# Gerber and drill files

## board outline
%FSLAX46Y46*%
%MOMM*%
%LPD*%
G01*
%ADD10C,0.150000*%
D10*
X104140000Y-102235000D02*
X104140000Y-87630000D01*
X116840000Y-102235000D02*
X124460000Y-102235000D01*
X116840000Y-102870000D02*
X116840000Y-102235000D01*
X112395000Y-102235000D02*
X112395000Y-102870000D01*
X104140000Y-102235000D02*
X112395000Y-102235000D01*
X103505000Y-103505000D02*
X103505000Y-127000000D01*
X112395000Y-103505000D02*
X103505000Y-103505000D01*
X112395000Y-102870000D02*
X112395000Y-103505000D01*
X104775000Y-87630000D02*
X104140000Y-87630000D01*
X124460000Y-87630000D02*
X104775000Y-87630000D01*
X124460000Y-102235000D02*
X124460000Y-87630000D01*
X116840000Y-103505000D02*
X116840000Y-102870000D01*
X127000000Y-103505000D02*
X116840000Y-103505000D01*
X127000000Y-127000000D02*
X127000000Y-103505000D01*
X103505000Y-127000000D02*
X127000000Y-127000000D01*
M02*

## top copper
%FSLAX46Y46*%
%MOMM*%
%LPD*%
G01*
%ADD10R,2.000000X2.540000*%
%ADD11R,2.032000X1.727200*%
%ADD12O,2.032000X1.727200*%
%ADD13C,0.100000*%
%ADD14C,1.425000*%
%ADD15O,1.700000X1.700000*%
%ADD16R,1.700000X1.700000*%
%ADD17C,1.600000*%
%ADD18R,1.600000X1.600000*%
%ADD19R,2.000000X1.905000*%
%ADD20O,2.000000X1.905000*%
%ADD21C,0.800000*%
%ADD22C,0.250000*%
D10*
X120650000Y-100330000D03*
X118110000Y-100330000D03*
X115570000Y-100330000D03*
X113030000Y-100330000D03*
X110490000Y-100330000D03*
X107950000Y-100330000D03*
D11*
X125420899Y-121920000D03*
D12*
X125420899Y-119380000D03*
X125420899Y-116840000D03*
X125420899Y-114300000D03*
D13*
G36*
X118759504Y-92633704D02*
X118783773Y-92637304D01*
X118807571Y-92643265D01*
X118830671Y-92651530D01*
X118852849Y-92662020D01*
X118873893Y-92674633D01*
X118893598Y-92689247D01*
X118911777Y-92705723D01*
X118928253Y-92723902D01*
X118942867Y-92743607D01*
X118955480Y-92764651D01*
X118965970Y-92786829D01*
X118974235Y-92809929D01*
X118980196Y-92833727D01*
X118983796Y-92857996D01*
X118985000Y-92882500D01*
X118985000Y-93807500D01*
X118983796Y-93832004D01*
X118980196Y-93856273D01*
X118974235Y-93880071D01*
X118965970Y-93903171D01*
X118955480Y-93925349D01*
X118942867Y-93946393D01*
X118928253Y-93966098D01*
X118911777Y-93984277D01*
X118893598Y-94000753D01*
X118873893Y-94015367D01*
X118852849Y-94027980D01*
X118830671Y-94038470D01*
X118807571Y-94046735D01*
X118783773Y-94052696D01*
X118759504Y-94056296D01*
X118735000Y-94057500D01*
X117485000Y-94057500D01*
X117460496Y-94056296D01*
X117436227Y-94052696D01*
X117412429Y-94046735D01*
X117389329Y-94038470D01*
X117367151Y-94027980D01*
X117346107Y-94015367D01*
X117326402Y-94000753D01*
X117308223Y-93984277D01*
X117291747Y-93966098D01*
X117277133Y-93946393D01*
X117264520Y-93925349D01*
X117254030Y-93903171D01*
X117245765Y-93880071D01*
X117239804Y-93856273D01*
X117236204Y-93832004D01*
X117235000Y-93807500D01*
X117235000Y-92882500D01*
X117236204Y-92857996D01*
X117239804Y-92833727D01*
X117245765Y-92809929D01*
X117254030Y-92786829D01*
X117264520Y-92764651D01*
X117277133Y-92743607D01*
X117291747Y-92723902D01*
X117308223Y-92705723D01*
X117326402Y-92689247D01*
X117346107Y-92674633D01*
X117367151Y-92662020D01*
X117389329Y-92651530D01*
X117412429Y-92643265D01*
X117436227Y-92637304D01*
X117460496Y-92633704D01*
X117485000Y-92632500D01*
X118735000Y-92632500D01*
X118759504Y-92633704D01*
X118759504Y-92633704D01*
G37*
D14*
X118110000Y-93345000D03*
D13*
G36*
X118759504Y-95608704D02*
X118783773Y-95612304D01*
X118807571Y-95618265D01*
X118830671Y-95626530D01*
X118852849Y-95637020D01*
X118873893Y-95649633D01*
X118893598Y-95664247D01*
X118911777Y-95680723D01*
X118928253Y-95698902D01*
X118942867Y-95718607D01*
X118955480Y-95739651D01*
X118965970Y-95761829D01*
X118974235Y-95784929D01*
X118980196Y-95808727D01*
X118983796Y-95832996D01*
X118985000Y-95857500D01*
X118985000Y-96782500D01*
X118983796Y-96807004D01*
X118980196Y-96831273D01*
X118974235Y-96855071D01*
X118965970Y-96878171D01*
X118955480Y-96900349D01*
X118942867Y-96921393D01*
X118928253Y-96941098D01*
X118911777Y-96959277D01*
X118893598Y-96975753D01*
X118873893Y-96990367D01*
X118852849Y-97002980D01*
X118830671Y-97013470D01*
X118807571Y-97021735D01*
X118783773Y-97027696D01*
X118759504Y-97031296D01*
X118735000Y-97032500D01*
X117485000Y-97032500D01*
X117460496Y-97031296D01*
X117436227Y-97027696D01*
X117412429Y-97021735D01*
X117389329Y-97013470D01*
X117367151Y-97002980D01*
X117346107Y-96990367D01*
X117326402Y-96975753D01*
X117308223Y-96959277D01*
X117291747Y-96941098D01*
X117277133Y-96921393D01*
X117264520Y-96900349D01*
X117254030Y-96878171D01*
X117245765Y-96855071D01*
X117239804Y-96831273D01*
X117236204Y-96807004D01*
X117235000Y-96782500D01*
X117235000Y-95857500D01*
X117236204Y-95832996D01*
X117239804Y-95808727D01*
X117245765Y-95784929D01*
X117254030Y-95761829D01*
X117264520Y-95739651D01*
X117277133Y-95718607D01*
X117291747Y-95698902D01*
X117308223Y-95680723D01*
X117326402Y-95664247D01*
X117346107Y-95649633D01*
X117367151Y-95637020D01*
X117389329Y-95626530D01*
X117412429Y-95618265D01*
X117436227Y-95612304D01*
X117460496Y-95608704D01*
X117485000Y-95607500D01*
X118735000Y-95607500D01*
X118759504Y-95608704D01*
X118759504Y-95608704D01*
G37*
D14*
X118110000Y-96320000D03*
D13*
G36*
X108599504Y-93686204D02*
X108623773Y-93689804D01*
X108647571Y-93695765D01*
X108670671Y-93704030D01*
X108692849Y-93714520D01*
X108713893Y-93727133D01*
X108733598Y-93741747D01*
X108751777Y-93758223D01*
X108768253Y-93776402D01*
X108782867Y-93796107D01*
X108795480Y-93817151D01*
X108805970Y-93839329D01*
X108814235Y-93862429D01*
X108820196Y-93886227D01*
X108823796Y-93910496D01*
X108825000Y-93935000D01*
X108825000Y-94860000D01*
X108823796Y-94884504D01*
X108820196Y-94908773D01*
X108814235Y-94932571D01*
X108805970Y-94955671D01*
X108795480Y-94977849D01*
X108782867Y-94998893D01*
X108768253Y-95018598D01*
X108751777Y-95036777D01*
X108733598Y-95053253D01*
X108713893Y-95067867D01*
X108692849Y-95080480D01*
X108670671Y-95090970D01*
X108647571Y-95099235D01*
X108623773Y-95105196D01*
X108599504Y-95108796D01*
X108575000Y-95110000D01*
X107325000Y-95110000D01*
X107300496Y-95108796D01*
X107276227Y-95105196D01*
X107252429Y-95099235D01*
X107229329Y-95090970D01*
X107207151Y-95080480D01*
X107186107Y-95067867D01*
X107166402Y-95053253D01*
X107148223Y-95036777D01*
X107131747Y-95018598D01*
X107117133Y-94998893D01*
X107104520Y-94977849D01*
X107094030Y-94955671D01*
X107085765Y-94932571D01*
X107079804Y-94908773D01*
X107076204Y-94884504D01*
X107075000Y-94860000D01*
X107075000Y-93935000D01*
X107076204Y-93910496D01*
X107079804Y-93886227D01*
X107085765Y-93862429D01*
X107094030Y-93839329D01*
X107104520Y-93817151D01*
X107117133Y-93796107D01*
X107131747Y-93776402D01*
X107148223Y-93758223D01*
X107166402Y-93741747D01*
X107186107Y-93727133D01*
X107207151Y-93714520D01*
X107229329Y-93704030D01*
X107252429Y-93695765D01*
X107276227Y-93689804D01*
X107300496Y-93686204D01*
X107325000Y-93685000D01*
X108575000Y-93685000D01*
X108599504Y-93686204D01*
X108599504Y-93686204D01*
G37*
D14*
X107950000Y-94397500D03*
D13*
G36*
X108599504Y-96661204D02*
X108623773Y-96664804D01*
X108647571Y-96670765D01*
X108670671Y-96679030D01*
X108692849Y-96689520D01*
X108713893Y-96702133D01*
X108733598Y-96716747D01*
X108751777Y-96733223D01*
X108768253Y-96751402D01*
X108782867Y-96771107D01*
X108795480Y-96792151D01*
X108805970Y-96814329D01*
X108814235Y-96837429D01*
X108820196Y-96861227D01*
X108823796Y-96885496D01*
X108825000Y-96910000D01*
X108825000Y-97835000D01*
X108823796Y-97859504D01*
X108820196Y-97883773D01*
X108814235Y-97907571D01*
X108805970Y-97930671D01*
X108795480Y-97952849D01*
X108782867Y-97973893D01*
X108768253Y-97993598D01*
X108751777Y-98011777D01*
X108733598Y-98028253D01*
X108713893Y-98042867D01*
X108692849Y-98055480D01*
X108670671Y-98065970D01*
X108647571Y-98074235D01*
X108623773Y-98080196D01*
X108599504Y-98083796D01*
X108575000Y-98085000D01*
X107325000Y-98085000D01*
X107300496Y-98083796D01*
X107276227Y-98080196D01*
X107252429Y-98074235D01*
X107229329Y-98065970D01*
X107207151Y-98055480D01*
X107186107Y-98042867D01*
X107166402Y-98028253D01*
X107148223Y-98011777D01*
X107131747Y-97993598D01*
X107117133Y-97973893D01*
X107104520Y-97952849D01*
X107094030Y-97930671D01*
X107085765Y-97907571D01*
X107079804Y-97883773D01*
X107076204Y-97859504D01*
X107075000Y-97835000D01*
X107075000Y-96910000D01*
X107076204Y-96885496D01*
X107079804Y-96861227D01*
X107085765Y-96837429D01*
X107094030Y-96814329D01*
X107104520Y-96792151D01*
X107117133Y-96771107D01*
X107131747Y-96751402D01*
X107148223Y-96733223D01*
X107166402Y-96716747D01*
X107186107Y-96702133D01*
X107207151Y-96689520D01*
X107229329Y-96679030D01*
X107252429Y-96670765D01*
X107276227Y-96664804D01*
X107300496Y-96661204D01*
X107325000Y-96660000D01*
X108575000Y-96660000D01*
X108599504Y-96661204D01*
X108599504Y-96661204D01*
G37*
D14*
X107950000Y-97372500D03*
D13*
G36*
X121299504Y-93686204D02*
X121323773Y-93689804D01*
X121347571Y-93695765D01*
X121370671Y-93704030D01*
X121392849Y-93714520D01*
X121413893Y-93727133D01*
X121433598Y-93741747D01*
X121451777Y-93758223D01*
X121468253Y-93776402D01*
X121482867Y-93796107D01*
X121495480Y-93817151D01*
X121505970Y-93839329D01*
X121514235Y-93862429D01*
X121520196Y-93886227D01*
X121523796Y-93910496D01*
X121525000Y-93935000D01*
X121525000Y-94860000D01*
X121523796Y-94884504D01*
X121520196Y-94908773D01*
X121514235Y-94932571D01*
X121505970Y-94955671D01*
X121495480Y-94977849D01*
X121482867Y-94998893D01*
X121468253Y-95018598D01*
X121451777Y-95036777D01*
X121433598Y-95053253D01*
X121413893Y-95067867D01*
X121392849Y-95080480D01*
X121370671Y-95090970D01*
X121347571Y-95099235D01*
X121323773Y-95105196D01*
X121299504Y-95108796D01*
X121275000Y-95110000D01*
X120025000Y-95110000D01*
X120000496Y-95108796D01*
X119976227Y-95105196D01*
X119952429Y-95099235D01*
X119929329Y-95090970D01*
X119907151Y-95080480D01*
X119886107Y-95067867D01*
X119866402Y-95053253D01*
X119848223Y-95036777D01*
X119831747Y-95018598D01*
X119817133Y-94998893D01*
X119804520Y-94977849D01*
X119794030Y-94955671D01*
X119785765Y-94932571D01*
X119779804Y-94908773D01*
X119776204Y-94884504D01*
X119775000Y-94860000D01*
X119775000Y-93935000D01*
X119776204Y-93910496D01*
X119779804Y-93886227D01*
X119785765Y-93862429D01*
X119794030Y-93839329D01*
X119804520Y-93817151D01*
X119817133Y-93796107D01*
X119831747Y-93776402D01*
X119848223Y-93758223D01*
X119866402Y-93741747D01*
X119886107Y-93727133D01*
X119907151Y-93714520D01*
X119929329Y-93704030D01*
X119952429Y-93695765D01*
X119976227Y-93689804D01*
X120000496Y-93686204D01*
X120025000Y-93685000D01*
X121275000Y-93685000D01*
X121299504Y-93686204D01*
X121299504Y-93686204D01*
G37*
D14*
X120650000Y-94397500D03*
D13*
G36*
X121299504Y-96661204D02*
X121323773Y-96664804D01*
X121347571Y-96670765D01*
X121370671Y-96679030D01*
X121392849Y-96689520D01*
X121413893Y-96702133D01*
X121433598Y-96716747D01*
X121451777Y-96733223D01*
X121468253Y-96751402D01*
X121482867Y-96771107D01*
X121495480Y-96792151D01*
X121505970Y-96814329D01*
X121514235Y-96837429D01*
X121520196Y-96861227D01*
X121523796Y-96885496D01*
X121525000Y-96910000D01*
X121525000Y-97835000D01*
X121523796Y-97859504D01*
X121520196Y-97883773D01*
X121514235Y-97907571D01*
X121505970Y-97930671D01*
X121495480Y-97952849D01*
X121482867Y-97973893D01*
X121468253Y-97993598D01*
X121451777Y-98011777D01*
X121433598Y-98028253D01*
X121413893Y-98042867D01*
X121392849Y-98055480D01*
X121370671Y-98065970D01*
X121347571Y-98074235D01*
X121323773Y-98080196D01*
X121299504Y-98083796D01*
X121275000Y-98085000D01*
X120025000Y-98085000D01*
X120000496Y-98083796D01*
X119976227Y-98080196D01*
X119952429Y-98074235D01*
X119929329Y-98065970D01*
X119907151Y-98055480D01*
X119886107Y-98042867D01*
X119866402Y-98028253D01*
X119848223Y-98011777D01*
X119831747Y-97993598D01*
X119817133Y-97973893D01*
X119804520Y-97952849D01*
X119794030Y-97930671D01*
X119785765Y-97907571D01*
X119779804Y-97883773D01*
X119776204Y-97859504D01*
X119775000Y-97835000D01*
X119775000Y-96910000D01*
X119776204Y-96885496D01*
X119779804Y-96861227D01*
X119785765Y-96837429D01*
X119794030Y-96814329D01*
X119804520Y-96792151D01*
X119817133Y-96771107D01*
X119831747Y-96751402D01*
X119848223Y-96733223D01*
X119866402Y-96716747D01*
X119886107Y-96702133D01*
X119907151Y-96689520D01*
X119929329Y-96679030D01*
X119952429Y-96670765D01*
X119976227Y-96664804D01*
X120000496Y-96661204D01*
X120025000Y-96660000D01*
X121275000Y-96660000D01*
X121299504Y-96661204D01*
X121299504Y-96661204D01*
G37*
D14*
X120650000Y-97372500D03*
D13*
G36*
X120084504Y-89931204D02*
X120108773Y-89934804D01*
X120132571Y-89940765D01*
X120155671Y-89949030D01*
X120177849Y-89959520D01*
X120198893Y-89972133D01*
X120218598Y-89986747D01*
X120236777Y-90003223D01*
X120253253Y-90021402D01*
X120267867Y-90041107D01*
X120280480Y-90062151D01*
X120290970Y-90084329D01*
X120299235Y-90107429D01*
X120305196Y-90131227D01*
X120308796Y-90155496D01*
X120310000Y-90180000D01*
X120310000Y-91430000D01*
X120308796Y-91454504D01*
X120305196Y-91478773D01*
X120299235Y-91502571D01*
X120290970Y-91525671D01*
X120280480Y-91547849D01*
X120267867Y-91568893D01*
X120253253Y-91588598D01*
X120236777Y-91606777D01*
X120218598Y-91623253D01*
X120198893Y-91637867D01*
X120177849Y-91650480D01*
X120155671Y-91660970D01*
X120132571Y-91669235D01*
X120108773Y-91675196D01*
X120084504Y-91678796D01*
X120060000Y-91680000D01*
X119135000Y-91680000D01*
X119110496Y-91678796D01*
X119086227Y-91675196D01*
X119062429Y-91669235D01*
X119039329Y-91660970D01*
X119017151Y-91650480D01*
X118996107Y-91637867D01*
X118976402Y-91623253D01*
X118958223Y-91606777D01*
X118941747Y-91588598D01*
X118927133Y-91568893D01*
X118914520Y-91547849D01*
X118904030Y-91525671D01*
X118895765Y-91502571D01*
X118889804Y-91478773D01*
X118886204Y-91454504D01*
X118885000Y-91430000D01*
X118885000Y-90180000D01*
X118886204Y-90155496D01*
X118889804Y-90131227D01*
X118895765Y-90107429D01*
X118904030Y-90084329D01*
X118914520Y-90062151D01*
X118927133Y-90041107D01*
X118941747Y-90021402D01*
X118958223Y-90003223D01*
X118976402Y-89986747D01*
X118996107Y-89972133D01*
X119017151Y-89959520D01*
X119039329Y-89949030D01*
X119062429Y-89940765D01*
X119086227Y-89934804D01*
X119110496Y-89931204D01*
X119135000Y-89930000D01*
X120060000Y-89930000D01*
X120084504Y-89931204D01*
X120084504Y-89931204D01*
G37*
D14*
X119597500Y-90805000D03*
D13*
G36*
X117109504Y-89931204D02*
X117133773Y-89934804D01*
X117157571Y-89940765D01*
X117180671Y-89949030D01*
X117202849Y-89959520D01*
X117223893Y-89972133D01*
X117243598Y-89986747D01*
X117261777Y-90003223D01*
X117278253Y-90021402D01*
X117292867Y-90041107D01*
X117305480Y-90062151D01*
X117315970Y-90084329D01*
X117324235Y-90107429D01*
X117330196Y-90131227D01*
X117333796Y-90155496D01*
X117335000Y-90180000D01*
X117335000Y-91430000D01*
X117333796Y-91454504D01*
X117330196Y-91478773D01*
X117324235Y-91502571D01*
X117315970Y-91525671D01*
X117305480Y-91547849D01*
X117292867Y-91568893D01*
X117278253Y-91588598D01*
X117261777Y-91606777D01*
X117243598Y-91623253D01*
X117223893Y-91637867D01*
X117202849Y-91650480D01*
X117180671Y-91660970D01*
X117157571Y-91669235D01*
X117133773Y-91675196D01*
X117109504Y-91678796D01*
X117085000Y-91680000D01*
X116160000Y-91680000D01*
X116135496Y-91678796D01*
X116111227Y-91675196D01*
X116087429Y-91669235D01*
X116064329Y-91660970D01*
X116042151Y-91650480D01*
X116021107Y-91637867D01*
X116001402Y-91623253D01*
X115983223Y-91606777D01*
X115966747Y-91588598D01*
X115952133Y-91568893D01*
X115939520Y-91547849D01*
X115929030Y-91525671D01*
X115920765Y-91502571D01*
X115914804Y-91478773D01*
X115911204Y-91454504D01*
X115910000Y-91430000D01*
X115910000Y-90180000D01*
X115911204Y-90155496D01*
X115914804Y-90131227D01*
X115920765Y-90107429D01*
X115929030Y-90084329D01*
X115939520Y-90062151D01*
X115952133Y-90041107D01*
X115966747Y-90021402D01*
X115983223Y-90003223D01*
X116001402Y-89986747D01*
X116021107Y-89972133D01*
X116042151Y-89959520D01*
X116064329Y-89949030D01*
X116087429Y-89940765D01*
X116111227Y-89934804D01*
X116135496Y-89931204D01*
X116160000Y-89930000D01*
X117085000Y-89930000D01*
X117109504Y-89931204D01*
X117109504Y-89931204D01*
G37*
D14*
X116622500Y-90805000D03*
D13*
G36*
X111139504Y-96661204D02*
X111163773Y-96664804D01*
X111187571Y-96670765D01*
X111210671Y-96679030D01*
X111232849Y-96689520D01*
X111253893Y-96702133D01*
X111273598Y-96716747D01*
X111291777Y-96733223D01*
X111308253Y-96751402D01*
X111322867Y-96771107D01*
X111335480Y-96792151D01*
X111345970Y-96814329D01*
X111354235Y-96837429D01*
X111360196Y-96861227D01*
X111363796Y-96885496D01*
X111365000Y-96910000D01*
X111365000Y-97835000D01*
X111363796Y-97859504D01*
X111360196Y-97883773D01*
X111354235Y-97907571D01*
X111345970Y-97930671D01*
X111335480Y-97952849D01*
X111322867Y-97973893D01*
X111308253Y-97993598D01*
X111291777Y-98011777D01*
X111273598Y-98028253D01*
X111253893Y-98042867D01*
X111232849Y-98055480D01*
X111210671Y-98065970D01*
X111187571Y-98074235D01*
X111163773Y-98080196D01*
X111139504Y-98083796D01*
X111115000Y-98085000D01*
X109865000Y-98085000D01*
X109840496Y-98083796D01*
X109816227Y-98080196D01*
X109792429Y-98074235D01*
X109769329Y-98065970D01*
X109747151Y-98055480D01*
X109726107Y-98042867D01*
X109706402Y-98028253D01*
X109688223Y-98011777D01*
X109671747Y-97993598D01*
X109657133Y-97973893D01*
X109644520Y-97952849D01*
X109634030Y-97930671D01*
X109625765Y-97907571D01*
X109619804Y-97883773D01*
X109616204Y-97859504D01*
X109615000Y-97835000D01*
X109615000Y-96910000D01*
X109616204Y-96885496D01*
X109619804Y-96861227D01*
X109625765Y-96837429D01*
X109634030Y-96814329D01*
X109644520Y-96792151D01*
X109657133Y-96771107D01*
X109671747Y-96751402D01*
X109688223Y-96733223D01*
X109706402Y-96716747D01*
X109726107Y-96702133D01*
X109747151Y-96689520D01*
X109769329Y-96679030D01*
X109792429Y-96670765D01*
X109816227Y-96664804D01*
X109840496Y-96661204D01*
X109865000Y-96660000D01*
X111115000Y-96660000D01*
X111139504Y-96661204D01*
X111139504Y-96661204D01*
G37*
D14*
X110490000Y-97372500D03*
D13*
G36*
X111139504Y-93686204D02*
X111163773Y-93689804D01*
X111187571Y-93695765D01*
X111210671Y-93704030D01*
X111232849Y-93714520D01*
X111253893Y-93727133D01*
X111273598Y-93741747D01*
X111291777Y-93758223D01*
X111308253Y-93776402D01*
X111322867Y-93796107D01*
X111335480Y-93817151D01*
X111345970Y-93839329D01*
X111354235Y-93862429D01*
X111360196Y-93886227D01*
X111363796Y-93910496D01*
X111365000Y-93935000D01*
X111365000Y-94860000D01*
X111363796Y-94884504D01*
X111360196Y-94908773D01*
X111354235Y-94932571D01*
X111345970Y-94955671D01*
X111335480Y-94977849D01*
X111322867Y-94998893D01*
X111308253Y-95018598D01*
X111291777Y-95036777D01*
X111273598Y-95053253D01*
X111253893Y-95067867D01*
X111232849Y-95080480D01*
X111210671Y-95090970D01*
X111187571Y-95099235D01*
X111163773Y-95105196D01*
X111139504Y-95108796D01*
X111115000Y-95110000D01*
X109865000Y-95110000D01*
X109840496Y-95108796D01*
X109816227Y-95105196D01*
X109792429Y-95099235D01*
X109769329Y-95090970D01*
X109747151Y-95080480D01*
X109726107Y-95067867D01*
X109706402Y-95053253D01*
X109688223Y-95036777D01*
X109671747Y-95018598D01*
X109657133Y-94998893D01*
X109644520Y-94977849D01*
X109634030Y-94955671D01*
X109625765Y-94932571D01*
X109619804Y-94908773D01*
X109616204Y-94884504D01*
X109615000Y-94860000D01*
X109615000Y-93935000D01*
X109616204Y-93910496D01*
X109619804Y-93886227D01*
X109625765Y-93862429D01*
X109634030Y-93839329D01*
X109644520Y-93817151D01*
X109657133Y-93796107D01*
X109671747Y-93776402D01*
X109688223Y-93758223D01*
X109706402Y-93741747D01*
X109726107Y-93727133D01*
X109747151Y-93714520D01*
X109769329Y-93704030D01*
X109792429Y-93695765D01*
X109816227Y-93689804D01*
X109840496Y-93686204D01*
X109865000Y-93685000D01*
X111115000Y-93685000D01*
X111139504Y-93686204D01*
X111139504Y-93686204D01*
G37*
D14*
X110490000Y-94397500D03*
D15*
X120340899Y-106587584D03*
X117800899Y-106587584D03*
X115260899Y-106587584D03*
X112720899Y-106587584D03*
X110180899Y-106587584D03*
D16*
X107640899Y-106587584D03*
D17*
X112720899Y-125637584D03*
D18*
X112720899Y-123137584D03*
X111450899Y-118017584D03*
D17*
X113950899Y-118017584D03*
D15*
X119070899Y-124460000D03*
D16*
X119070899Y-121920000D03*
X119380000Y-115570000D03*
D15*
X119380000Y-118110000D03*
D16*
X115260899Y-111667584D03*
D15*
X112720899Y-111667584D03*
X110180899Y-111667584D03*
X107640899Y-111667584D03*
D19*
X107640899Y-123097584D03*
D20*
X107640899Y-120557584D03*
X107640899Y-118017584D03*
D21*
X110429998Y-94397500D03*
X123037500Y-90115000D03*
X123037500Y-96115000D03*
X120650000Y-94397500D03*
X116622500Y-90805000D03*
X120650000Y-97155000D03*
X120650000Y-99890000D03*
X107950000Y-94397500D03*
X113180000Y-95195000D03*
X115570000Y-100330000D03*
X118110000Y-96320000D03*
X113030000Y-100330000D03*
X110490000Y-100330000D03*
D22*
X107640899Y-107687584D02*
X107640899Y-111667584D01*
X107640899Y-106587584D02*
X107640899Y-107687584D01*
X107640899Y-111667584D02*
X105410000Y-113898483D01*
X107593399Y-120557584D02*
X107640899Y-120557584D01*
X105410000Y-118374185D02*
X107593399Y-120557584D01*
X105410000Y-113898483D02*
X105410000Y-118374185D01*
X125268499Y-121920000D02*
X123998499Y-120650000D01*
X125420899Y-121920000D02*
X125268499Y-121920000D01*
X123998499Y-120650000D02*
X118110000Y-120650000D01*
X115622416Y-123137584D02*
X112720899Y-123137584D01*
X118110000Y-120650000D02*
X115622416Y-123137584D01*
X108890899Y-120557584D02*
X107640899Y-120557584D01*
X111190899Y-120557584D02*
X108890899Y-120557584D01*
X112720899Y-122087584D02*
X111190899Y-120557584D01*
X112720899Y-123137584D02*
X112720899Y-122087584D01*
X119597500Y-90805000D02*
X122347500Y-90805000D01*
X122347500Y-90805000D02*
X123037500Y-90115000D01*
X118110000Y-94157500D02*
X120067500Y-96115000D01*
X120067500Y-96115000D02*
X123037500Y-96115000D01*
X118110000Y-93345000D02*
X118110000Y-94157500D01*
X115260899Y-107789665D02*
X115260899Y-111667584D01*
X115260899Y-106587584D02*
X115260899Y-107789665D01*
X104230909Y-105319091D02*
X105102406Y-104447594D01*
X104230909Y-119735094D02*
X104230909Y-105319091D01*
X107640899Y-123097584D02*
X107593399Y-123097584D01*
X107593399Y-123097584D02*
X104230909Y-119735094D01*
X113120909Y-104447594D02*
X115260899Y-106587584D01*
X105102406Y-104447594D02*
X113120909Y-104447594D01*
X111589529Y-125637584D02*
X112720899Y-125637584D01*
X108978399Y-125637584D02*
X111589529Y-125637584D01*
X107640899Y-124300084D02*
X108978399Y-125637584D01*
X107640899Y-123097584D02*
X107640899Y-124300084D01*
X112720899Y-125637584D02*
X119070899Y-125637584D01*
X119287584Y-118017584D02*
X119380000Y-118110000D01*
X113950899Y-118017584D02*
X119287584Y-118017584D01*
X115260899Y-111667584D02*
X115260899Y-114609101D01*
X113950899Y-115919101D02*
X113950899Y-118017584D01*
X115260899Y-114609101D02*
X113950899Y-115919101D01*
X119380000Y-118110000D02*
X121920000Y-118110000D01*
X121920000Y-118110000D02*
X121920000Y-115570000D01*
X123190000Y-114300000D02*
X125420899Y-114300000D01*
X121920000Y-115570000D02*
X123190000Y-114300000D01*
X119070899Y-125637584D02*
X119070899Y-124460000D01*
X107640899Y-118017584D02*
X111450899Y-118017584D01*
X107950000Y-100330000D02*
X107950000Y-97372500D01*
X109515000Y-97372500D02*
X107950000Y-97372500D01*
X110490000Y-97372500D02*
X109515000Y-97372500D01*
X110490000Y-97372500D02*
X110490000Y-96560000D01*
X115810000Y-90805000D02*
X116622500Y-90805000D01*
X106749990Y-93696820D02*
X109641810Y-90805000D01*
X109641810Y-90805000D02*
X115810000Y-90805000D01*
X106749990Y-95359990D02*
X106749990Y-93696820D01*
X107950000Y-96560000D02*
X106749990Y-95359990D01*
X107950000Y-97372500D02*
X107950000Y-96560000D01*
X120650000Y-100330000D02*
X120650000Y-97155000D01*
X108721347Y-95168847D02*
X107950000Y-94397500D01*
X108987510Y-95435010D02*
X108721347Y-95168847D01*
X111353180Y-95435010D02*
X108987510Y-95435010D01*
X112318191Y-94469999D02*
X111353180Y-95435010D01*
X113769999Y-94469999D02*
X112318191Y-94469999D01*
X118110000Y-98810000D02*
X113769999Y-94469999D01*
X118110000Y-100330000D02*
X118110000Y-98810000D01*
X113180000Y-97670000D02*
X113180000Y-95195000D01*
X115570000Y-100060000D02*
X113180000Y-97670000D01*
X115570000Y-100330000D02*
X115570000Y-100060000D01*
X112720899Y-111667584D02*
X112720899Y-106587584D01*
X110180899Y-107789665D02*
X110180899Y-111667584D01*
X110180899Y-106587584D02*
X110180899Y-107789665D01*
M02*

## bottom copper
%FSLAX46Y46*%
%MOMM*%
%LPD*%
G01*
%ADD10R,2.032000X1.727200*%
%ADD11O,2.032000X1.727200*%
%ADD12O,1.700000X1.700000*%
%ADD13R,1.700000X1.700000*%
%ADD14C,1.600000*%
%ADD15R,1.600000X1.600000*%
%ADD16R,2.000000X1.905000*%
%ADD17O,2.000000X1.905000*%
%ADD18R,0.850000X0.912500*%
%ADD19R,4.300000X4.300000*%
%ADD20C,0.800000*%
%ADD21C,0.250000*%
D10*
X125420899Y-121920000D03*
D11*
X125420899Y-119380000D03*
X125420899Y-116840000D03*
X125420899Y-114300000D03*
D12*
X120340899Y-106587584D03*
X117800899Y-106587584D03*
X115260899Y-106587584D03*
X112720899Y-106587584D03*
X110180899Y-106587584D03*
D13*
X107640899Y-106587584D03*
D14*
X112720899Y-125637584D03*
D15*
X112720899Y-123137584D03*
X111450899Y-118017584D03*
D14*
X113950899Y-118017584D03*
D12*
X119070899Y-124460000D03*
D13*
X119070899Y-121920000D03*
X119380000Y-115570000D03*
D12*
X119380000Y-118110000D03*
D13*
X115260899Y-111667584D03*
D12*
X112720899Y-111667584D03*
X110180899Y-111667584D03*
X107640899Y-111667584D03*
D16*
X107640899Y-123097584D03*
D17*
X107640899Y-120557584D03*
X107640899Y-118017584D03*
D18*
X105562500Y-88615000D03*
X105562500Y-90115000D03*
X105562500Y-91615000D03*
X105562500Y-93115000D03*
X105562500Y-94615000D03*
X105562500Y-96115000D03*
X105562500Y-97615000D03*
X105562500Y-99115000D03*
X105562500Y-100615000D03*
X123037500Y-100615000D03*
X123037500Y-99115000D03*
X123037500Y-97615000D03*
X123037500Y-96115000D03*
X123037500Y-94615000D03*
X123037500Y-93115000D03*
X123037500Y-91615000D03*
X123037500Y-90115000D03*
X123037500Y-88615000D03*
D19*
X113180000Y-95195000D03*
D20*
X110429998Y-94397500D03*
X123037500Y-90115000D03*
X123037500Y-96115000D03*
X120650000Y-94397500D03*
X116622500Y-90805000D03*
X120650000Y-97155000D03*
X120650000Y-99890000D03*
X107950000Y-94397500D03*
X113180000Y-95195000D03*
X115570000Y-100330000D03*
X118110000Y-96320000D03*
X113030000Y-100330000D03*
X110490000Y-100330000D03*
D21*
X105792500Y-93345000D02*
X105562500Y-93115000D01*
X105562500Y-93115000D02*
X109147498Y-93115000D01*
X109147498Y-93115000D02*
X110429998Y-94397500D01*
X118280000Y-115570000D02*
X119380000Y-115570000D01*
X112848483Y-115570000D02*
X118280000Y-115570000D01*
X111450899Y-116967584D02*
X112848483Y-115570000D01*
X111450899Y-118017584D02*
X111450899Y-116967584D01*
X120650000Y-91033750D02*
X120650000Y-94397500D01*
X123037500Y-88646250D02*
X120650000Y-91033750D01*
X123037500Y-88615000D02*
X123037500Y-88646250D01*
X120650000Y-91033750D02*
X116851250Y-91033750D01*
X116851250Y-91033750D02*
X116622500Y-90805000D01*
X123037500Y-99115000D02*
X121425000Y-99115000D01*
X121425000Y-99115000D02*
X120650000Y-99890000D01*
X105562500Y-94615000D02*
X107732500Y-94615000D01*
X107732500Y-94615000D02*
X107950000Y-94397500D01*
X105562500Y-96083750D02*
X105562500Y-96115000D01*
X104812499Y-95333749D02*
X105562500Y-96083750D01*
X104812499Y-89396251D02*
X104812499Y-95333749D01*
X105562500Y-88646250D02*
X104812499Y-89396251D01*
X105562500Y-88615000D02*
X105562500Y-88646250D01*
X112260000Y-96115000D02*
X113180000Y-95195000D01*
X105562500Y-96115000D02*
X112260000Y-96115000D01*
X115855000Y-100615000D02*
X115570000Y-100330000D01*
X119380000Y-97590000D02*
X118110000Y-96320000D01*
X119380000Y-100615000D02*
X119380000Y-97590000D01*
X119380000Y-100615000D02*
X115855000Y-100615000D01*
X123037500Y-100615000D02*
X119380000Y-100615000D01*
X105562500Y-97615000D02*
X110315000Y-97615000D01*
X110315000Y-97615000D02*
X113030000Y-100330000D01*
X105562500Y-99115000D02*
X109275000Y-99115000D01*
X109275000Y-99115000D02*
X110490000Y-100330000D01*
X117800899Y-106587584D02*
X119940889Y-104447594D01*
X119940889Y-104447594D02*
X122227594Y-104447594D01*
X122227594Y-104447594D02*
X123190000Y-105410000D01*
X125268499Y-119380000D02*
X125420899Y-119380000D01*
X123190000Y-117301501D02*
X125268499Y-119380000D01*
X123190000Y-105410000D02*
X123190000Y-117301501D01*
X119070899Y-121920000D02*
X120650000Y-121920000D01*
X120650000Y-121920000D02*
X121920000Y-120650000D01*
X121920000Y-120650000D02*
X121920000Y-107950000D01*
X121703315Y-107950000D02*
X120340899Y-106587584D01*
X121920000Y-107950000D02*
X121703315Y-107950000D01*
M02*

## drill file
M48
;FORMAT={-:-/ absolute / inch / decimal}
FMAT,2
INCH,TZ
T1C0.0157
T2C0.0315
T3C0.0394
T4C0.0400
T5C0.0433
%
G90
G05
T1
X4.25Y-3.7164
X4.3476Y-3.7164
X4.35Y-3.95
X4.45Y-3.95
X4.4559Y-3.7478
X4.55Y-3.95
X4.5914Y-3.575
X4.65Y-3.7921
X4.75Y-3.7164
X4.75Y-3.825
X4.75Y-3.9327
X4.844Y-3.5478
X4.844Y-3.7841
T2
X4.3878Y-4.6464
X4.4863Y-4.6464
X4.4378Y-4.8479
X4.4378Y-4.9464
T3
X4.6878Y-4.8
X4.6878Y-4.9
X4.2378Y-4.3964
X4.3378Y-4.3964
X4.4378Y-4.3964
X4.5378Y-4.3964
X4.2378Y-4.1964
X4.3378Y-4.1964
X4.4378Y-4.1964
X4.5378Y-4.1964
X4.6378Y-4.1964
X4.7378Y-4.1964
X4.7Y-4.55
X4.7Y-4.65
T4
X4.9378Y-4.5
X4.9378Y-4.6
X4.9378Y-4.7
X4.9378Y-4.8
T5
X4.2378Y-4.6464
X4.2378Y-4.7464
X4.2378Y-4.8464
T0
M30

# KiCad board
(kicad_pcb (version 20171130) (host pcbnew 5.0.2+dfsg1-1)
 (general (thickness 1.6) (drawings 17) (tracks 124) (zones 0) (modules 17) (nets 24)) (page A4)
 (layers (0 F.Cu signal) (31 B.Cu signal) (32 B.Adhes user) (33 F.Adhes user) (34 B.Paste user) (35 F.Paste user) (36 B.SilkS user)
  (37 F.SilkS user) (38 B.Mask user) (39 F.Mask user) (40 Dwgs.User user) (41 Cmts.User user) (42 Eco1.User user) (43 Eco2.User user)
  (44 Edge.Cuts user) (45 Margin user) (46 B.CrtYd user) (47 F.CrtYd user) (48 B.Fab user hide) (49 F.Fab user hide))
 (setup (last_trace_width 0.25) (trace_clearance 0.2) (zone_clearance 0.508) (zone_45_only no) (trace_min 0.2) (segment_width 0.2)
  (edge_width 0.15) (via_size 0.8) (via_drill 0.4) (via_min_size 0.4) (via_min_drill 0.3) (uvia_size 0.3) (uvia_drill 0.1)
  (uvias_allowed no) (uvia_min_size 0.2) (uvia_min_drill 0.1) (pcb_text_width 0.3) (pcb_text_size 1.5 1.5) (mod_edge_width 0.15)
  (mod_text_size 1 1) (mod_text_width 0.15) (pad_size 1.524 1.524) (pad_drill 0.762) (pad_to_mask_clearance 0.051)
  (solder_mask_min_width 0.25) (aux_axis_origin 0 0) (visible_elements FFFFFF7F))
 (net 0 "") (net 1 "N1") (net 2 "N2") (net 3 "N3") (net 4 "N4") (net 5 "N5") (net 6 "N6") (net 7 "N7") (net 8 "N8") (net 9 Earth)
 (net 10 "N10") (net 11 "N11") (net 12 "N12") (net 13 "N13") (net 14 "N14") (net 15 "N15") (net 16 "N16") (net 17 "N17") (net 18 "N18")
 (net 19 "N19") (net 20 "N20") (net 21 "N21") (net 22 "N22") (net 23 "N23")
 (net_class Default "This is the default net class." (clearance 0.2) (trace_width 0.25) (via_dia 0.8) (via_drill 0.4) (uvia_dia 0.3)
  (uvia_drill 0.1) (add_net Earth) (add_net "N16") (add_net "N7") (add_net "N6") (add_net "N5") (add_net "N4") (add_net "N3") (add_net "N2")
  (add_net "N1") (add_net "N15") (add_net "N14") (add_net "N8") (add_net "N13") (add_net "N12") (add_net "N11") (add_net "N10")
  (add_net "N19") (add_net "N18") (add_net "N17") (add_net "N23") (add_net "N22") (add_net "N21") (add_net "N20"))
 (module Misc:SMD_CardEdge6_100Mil (layer F.Cu) (at 114.3 100.33)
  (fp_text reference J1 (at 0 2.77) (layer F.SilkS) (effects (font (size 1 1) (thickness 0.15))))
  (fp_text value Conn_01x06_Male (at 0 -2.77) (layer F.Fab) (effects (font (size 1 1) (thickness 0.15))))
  (pad 6 smd rect (at 6.35 0) (size 2 2.54) (layers F.Cu F.Paste F.Mask) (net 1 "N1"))
  (pad 5 smd rect (at 3.81 0) (size 2 2.54) (layers F.Cu F.Paste F.Mask) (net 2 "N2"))
  (pad 4 smd rect (at 1.27 0) (size 2 2.54) (layers F.Cu F.Paste F.Mask) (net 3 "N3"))
  (pad 3 smd rect (at -1.27 0) (size 2 2.54) (layers F.Cu F.Paste F.Mask) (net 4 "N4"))
  (pad 2 smd rect (at -3.81 0) (size 2 2.54) (layers F.Cu F.Paste F.Mask) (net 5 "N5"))
  (pad 1 smd rect (at -6.35 0) (size 2 2.54) (layers F.Cu F.Paste F.Mask) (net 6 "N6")))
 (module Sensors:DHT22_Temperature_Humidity (layer F.Cu) (at 125.420899 118.11 90)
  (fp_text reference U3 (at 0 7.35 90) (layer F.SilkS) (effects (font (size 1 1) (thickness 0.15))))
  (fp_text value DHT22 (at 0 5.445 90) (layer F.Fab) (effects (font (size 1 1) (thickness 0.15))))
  (pad 1 thru_hole rect (at -3.81 0 180) (size 2.032 1.7272) (drill 1.016) (layers *.Cu *.Mask F.SilkS) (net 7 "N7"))
  (pad 2 thru_hole oval (at -1.27 0 180) (size 2.032 1.7272) (drill 1.016) (layers *.Cu *.Mask F.SilkS) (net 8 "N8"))
  (pad 3 thru_hole oval (at 1.27 0 180) (size 2.032 1.7272) (drill 1.016) (layers *.Cu *.Mask F.SilkS))
  (pad 4 thru_hole oval (at 3.81 0 180) (size 2.032 1.7272) (drill 1.016) (layers *.Cu *.Mask F.SilkS) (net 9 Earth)))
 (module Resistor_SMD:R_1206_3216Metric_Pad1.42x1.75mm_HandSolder (layer F.Cu) (at 118.11 94.8325 270)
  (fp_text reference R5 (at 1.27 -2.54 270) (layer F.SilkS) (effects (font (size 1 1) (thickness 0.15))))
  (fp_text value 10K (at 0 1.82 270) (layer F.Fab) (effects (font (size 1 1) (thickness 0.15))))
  (pad 1 smd roundrect (at -1.4875 0 270) (size 1.425 1.75) (layers F.Cu F.Paste F.Mask) (roundrect_rratio 0.175439) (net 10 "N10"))
  (pad 2 smd roundrect (at 1.4875 0 270) (size 1.425 1.75) (layers F.Cu F.Paste F.Mask) (roundrect_rratio 0.175439) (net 3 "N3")))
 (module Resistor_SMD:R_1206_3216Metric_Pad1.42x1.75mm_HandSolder (layer F.Cu) (at 107.95 95.885 90)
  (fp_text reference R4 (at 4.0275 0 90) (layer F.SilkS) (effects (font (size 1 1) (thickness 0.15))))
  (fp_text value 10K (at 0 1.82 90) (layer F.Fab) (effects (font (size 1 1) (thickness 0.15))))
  (pad 2 smd roundrect (at 1.4875 0 90) (size 1.425 1.75) (layers F.Cu F.Paste F.Mask) (roundrect_rratio 0.175439) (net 2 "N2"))
  (pad 1 smd roundrect (at -1.4875 0 90) (size 1.425 1.75) (layers F.Cu F.Paste F.Mask) (roundrect_rratio 0.175439) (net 6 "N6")))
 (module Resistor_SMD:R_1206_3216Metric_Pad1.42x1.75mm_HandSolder (layer F.Cu) (at 120.65 95.885 270)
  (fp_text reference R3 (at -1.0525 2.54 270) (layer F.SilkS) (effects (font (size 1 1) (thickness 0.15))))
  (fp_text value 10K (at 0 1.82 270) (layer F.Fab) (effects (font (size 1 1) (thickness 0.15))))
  (pad 1 smd roundrect (at -1.4875 0 270) (size 1.425 1.75) (layers F.Cu F.Paste F.Mask) (roundrect_rratio 0.175439) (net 6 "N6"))
  (pad 2 smd roundrect (at 1.4875 0 270) (size 1.425 1.75) (layers F.Cu F.Paste F.Mask) (roundrect_rratio 0.175439) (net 1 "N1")))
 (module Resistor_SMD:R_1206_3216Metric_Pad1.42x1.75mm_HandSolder (layer F.Cu) (at 118.11 90.805)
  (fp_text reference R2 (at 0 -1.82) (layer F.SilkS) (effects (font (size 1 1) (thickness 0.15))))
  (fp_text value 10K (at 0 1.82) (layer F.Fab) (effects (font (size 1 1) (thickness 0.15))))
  (pad 2 smd roundrect (at 1.4875 0) (size 1.425 1.75) (layers F.Cu F.Paste F.Mask) (roundrect_rratio 0.175439) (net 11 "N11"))
  (pad 1 smd roundrect (at -1.4875 0) (size 1.425 1.75) (layers F.Cu F.Paste F.Mask) (roundrect_rratio 0.175439) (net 6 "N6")))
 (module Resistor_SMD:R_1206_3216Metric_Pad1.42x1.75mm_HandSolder (layer F.Cu) (at 110.49 95.885 90)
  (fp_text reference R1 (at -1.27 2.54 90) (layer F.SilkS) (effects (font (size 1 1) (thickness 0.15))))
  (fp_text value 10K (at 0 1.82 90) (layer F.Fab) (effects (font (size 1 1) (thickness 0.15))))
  (pad 1 smd roundrect (at -1.4875 0 90) (size 1.425 1.75) (layers F.Cu F.Paste F.Mask) (roundrect_rratio 0.175439) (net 6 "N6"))
  (pad 2 smd roundrect (at 1.4875 0 90) (size 1.425 1.75) (layers F.Cu F.Paste F.Mask) (roundrect_rratio 0.175439) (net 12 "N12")))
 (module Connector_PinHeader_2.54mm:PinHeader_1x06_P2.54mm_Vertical (layer F.Cu) (at 107.640899 106.587584 90)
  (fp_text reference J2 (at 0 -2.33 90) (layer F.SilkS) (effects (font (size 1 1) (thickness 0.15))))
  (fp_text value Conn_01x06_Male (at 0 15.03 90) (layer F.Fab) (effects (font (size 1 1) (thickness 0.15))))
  (pad 6 thru_hole oval (at 0 12.7 90) (size 1.7 1.7) (drill 1) (layers *.Cu *.Mask) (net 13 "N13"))
  (pad 5 thru_hole oval (at 0 10.16 90) (size 1.7 1.7) (drill 1) (layers *.Cu *.Mask) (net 8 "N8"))
  (pad 4 thru_hole oval (at 0 7.62 90) (size 1.7 1.7) (drill 1) (layers *.Cu *.Mask) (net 9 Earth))
  (pad 3 thru_hole oval (at 0 5.08 90) (size 1.7 1.7) (drill 1) (layers *.Cu *.Mask) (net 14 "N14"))
  (pad 2 thru_hole oval (at 0 2.54 90) (size 1.7 1.7) (drill 1) (layers *.Cu *.Mask) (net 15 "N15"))
  (pad 1 thru_hole rect (at 0 0 90) (size 1.7 1.7) (drill 1) (layers *.Cu *.Mask) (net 7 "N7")))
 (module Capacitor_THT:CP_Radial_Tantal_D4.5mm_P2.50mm (layer F.Cu) (at 112.720899 123.137584 270)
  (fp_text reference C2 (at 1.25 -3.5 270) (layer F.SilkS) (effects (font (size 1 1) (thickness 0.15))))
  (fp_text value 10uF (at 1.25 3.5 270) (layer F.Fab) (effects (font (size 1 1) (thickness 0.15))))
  (pad 2 thru_hole circle (at 2.5 0 270) (size 1.6 1.6) (drill 0.8) (layers *.Cu *.Mask) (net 9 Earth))
  (pad 1 thru_hole rect (at 0 0 270) (size 1.6 1.6) (drill 0.8) (layers *.Cu *.Mask) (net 7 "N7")))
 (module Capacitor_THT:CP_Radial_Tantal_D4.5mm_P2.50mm (layer F.Cu) (at 111.450899 118.017584)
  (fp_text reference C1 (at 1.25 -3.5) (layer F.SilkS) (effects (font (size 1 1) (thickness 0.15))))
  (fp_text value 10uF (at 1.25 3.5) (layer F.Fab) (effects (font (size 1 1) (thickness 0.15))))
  (pad 1 thru_hole rect (at 0 0) (size 1.6 1.6) (drill 0.8) (layers *.Cu *.Mask) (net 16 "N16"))
  (pad 2 thru_hole circle (at 2.5 0) (size 1.6 1.6) (drill 0.8) (layers *.Cu *.Mask) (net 9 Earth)))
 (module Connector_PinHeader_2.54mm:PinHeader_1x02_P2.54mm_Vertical (layer F.Cu) (at 119.070899 121.92)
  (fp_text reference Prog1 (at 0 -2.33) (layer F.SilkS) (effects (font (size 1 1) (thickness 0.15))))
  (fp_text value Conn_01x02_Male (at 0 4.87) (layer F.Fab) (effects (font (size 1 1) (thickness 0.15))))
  (pad 2 thru_hole oval (at 0 2.54) (size 1.7 1.7) (drill 1) (layers *.Cu *.Mask) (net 9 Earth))
  (pad 1 thru_hole rect (at 0 0) (size 1.7 1.7) (drill 1) (layers *.Cu *.Mask) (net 13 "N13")))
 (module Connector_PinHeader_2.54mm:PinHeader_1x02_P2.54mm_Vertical (layer F.Cu) (at 119.38 115.57)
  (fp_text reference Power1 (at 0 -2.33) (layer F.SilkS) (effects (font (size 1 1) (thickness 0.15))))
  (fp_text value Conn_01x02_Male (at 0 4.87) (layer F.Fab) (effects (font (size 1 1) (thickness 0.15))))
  (pad 1 thru_hole rect (at 0 0) (size 1.7 1.7) (drill 1) (layers *.Cu *.Mask) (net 16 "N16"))
  (pad 2 thru_hole oval (at 0 2.54) (size 1.7 1.7) (drill 1) (layers *.Cu *.Mask) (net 9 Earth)))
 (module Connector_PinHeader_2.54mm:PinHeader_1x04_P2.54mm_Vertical (layer F.Cu) (at 115.260899 111.667584 270)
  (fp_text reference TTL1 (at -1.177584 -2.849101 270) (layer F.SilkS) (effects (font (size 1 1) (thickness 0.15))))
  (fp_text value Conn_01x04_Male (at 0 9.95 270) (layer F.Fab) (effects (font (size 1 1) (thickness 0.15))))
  (pad 1 thru_hole rect (at 0 0 270) (size 1.7 1.7) (drill 1) (layers *.Cu *.Mask) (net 9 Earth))
  (pad 2 thru_hole oval (at 0 2.54 270) (size 1.7 1.7) (drill 1) (layers *.Cu *.Mask) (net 14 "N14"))
  (pad 3 thru_hole oval (at 0 5.08 270) (size 1.7 1.7) (drill 1) (layers *.Cu *.Mask) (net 15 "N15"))
  (pad 4 thru_hole oval (at 0 7.62 270) (size 1.7 1.7) (drill 1) (layers *.Cu *.Mask) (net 7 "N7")))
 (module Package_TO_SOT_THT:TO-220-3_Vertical (layer F.Cu) (at 107.640899 123.097584 90)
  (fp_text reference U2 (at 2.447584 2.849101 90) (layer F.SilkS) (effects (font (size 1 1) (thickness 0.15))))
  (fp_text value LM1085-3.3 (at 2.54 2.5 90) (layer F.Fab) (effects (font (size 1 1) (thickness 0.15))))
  (pad 1 thru_hole rect (at 0 0 90) (size 1.905 2) (drill 1.1) (layers *.Cu *.Mask) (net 9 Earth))
  (pad 2 thru_hole oval (at 2.54 0 90) (size 1.905 2) (drill 1.1) (layers *.Cu *.Mask) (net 7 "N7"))
  (pad 3 thru_hole oval (at 5.08 0 90) (size 1.905 2) (drill 1.1) (layers *.Cu *.Mask) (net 16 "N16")))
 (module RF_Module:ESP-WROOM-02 (layer B.Cu) (at 114.3 94.615 180)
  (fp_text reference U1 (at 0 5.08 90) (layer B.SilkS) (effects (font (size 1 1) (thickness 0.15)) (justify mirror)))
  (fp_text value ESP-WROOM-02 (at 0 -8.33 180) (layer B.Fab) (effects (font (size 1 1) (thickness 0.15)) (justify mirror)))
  (pad 18 smd rect (at 8.7375 6 180) (size 0.85 0.9125) (layers B.Cu B.Paste B.Mask) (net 3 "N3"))
  (pad 17 smd rect (at 8.7375 4.5 180) (size 0.85 0.9125) (layers B.Cu B.Paste B.Mask) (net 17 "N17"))
  (pad 16 smd rect (at 8.7375 3 180) (size 0.85 0.9125) (layers B.Cu B.Paste B.Mask) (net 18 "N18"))
  (pad 15 smd rect (at 8.7375 1.5 180) (size 0.85 0.9125) (layers B.Cu B.Paste B.Mask) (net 12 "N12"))
  (pad 14 smd rect (at 8.7375 0 180) (size 0.85 0.9125) (layers B.Cu B.Paste B.Mask) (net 2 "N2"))
  (pad 13 smd rect (at 8.7375 -1.5 180) (size 0.85 0.9125) (layers B.Cu B.Paste B.Mask) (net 3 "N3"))
  (pad 12 smd rect (at 8.7375 -3 180) (size 0.85 0.9125) (layers B.Cu B.Paste B.Mask) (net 4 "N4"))
  (pad 11 smd rect (at 8.7375 -4.5 180) (size 0.85 0.9125) (layers B.Cu B.Paste B.Mask) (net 5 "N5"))
  (pad 10 smd rect (at 8.7375 -6 180) (size 0.85 0.9125) (layers B.Cu B.Paste B.Mask) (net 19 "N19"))
  (pad 9 smd rect (at -8.7375 -6 180) (size 0.85 0.9125) (layers B.Cu B.Paste B.Mask) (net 3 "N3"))
  (pad 8 smd rect (at -8.7375 -4.5 180) (size 0.85 0.9125) (layers B.Cu B.Paste B.Mask) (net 1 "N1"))
  (pad 7 smd rect (at -8.7375 -3 180) (size 0.85 0.9125) (layers B.Cu B.Paste B.Mask) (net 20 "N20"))
  (pad 6 smd rect (at -8.7375 -1.5 180) (size 0.85 0.9125) (layers B.Cu B.Paste B.Mask) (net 10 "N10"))
  (pad 5 smd rect (at -8.7375 0 180) (size 0.85 0.9125) (layers B.Cu B.Paste B.Mask) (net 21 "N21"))
  (pad 4 smd rect (at -8.7375 1.5 180) (size 0.85 0.9125) (layers B.Cu B.Paste B.Mask) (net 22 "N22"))
  (pad 3 smd rect (at -8.7375 3 180) (size 0.85 0.9125) (layers B.Cu B.Paste B.Mask) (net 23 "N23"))
  (pad 2 smd rect (at -8.7375 4.5 180) (size 0.85 0.9125) (layers B.Cu B.Paste B.Mask) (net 11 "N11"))
  (pad 1 smd rect (at -8.7375 6 180) (size 0.85 0.9125) (layers B.Cu B.Paste B.Mask) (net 6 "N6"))
  (pad 19 smd rect (at 1.12 -0.58 180) (size 4.3 4.3) (layers B.Cu B.Paste B.Mask) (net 3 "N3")))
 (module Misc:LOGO (layer B.Cu) (at 122.555 111.125 180)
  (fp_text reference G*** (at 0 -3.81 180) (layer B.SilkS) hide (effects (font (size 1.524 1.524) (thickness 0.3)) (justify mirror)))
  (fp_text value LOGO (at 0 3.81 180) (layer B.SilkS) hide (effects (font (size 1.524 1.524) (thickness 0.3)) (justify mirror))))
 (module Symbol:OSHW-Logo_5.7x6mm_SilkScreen (layer B.Cu) (at 121.92 123.825 180)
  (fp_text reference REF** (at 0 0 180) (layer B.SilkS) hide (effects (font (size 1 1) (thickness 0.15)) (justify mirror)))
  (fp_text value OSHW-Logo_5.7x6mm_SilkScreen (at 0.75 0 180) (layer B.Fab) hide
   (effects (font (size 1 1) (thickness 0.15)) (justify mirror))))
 (gr_line (start 104.14 102.235) (end 104.14 87.63) (layer Edge.Cuts) (width 0.15))
 (gr_line (start 116.84 102.235) (end 124.46 102.235) (layer Edge.Cuts) (width 0.15))
 (gr_line (start 116.84 102.87) (end 116.84 102.235) (layer Edge.Cuts) (width 0.15))
 (gr_line (start 112.395 102.235) (end 112.395 102.87) (layer Edge.Cuts) (width 0.15))
 (gr_line (start 104.14 102.235) (end 112.395 102.235) (layer Edge.Cuts) (width 0.15))
 (gr_line (start 103.505 103.505) (end 103.505 127) (layer Edge.Cuts) (width 0.15))
 (gr_line (start 112.395 103.505) (end 103.505 103.505) (layer Edge.Cuts) (width 0.15))
 (gr_line (start 112.395 102.87) (end 112.395 103.505) (layer Edge.Cuts) (width 0.15))
 (gr_line (start 104.775 87.63) (end 104.14 87.63) (layer Edge.Cuts) (width 0.15))
 (gr_line (start 124.46 87.63) (end 104.775 87.63) (layer Edge.Cuts) (width 0.15))
 (gr_line (start 124.46 102.235) (end 124.46 87.63) (layer Edge.Cuts) (width 0.15))
 (gr_line (start 116.84 103.505) (end 116.84 102.87) (layer Edge.Cuts) (width 0.15))
 (gr_line (start 127 103.505) (end 116.84 103.505) (layer Edge.Cuts) (width 0.15))
 (gr_line (start 127 127) (end 127 103.505) (layer Edge.Cuts) (width 0.15))
 (gr_line (start 103.505 127) (end 127 127) (layer Edge.Cuts) (width 0.15))
 (segment (start 107.640899 107.687584) (end 107.640899 111.667584) (width 0.25) (layer F.Cu) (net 7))
 (segment (start 107.640899 106.587584) (end 107.640899 107.687584) (width 0.25) (layer F.Cu) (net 7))
 (segment (start 107.640899 111.667584) (end 105.41 113.898483) (width 0.25) (layer F.Cu) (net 7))
 (segment (start 107.593399 120.557584) (end 107.640899 120.557584) (width 0.25) (layer F.Cu) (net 7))
 (segment (start 105.41 118.374185) (end 107.593399 120.557584) (width 0.25) (layer F.Cu) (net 7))
 (segment (start 105.41 113.898483) (end 105.41 118.374185) (width 0.25) (layer F.Cu) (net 7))
 (segment (start 125.268499 121.92) (end 123.998499 120.65) (width 0.25) (layer F.Cu) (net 7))
 (segment (start 125.420899 121.92) (end 125.268499 121.92) (width 0.25) (layer F.Cu) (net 7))
 (segment (start 123.998499 120.65) (end 118.11 120.65) (width 0.25) (layer F.Cu) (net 7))
 (segment (start 115.622416 123.137584) (end 112.720899 123.137584) (width 0.25) (layer F.Cu) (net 7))
 (segment (start 118.11 120.65) (end 115.622416 123.137584) (width 0.25) (layer F.Cu) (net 7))
 (segment (start 108.890899 120.557584) (end 107.640899 120.557584) (width 0.25) (layer F.Cu) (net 7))
 (segment (start 111.190899 120.557584) (end 108.890899 120.557584) (width 0.25) (layer F.Cu) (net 7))
 (segment (start 112.720899 122.087584) (end 111.190899 120.557584) (width 0.25) (layer F.Cu) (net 7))
 (segment (start 112.720899 123.137584) (end 112.720899 122.087584) (width 0.25) (layer F.Cu) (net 7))
 (segment (start 105.7925 93.345) (end 105.5625 93.115) (width 0.25) (layer B.Cu) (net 12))
 (via (at 110.429998 94.3975) (size 0.8) (drill 0.4) (layers F.Cu B.Cu) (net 12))
 (segment (start 105.5625 93.115) (end 109.147498 93.115) (width 0.25) (layer B.Cu) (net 12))
 (segment (start 109.147498 93.115) (end 110.429998 94.3975) (width 0.25) (layer B.Cu) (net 12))
 (via (at 123.0375 90.115) (size 0.8) (drill 0.4) (layers F.Cu B.Cu) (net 11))
 (segment (start 119.5975 90.805) (end 122.3475 90.805) (width 0.25) (layer F.Cu) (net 11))
 (segment (start 122.3475 90.805) (end 123.0375 90.115) (width 0.25) (layer F.Cu) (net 11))
 (via (at 123.0375 96.115) (size 0.8) (drill 0.4) (layers F.Cu B.Cu) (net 10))
 (segment (start 118.11 94.1575) (end 120.0675 96.115) (width 0.25) (layer F.Cu) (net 10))
 (segment (start 120.0675 96.115) (end 123.0375 96.115) (width 0.25) (layer F.Cu) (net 10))
 (segment (start 118.11 93.345) (end 118.11 94.1575) (width 0.25) (layer F.Cu) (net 10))
 (segment (start 115.260899 107.789665) (end 115.260899 111.667584) (width 0.25) (layer F.Cu) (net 9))
 (segment (start 115.260899 106.587584) (end 115.260899 107.789665) (width 0.25) (layer F.Cu) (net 9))
 (segment (start 104.230909 105.319091) (end 105.102406 104.447594) (width 0.25) (layer F.Cu) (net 9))
 (segment (start 104.230909 119.735094) (end 104.230909 105.319091) (width 0.25) (layer F.Cu) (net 9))
 (segment (start 107.640899 123.097584) (end 107.593399 123.097584) (width 0.25) (layer F.Cu) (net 9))
 (segment (start 107.593399 123.097584) (end 104.230909 119.735094) (width 0.25) (layer F.Cu) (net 9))
 (segment (start 113.120909 104.447594) (end 115.260899 106.587584) (width 0.25) (layer F.Cu) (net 9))
 (segment (start 105.102406 104.447594) (end 113.120909 104.447594) (width 0.25) (layer F.Cu) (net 9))
 (segment (start 111.589529 125.637584) (end 112.720899 125.637584) (width 0.25) (layer F.Cu) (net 9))
 (segment (start 108.978399 125.637584) (end 111.589529 125.637584) (width 0.25) (layer F.Cu) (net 9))
 (segment (start 107.640899 124.300084) (end 108.978399 125.637584) (width 0.25) (layer F.Cu) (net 9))
 (segment (start 107.640899 123.097584) (end 107.640899 124.300084) (width 0.25) (layer F.Cu) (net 9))
 (segment (start 112.720899 125.637584) (end 119.070899 125.637584) (width 0.25) (layer F.Cu) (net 9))
 (segment (start 119.287584 118.017584) (end 119.38 118.11) (width 0.25) (layer F.Cu) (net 9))
 (segment (start 113.950899 118.017584) (end 119.287584 118.017584) (width 0.25) (layer F.Cu) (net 9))
 (segment (start 115.260899 111.667584) (end 115.260899 114.609101) (width 0.25) (layer F.Cu) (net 9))
 (segment (start 113.950899 115.919101) (end 113.950899 118.017584) (width 0.25) (layer F.Cu) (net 9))
 (segment (start 115.260899 114.609101) (end 113.950899 115.919101) (width 0.25) (layer F.Cu) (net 9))
 (segment (start 119.38 118.11) (end 121.92 118.11) (width 0.25) (layer F.Cu) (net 9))
 (segment (start 121.92 118.11) (end 121.92 115.57) (width 0.25) (layer F.Cu) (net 9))
 (segment (start 123.19 114.3) (end 125.420899 114.3) (width 0.25) (layer F.Cu) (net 9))
 (segment (start 121.92 115.57) (end 123.19 114.3) (width 0.25) (layer F.Cu) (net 9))
 (segment (start 119.070899 125.637584) (end 119.070899 124.46) (width 0.25) (layer F.Cu) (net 9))
 (segment (start 107.640899 118.017584) (end 111.450899 118.017584) (width 0.25) (layer F.Cu) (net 16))
 (segment (start 118.28 115.57) (end 119.38 115.57) (width 0.25) (layer B.Cu) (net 16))
 (segment (start 112.848483 115.57) (end 118.28 115.57) (width 0.25) (layer B.Cu) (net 16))
 (segment (start 111.450899 116.967584) (end 112.848483 115.57) (width 0.25) (layer B.Cu) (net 16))
 (segment (start 111.450899 118.017584) (end 111.450899 116.967584) (width 0.25) (layer B.Cu) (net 16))
 (segment (start 107.95 100.33) (end 107.95 97.3725) (width 0.25) (layer F.Cu) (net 6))
 (segment (start 109.515 97.3725) (end 107.95 97.3725) (width 0.25) (layer F.Cu) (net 6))
 (segment (start 110.49 97.3725) (end 109.515 97.3725) (width 0.25) (layer F.Cu) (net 6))
 (via (at 120.65 94.3975) (size 0.8) (drill 0.4) (layers F.Cu B.Cu) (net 6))
 (segment (start 120.65 91.03375) (end 120.65 94.3975) (width 0.25) (layer B.Cu) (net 6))
 (segment (start 123.0375 88.64625) (end 120.65 91.03375) (width 0.25) (layer B.Cu) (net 6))
 (segment (start 123.0375 88.615) (end 123.0375 88.64625) (width 0.25) (layer B.Cu) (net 6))
 (via (at 116.6225 90.805) (size 0.8) (drill 0.4) (layers F.Cu B.Cu) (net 6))
 (segment (start 120.65 91.03375) (end 116.85125 91.03375) (width 0.25) (layer B.Cu) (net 6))
 (segment (start 116.85125 91.03375) (end 116.6225 90.805) (width 0.25) (layer B.Cu) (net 6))
 (segment (start 110.49 97.3725) (end 110.49 96.56) (width 0.25) (layer F.Cu) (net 6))
 (segment (start 115.81 90.805) (end 116.6225 90.805) (width 0.25) (layer F.Cu) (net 6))
 (segment (start 106.74999 93.69682) (end 109.64181 90.805) (width 0.25) (layer F.Cu) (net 6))
 (segment (start 109.64181 90.805) (end 115.81 90.805) (width 0.25) (layer F.Cu) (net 6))
 (segment (start 106.74999 95.35999) (end 106.74999 93.69682) (width 0.25) (layer F.Cu) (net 6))
 (segment (start 107.95 96.56) (end 106.74999 95.35999) (width 0.25) (layer F.Cu) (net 6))
 (segment (start 107.95 97.3725) (end 107.95 96.56) (width 0.25) (layer F.Cu) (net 6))
 (via (at 120.65 97.155) (size 0.8) (drill 0.4) (layers F.Cu B.Cu) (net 1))
 (segment (start 120.65 100.33) (end 120.65 97.155) (width 0.25) (layer F.Cu) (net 1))
 (via (at 120.65 99.89) (size 0.8) (drill 0.4) (layers F.Cu B.Cu) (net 1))
 (segment (start 123.0375 99.115) (end 121.425 99.115) (width 0.25) (layer B.Cu) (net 1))
 (segment (start 121.425 99.115) (end 120.65 99.89) (width 0.25) (layer B.Cu) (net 1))
 (via (at 107.95 94.3975) (size 0.8) (drill 0.4) (layers F.Cu B.Cu) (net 2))
 (segment (start 105.5625 94.615) (end 107.7325 94.615) (width 0.25) (layer B.Cu) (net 2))
 (segment (start 107.7325 94.615) (end 107.95 94.3975) (width 0.25) (layer B.Cu) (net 2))
 (segment (start 108.721347 95.168847) (end 107.95 94.3975) (width 0.25) (layer F.Cu) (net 2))
 (segment (start 108.98751 95.43501) (end 108.721347 95.168847) (width 0.25) (layer F.Cu) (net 2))
 (segment (start 111.35318 95.43501) (end 108.98751 95.43501) (width 0.25) (layer F.Cu) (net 2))
 (segment (start 112.318191 94.469999) (end 111.35318 95.43501) (width 0.25) (layer F.Cu) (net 2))
 (segment (start 113.769999 94.469999) (end 112.318191 94.469999) (width 0.25) (layer F.Cu) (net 2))
 (segment (start 118.11 98.81) (end 113.769999 94.469999) (width 0.25) (layer F.Cu) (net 2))
 (segment (start 118.11 100.33) (end 118.11 98.81) (width 0.25) (layer F.Cu) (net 2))
 (segment (start 105.5625 96.08375) (end 105.5625 96.115) (width 0.25) (layer B.Cu) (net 3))
 (segment (start 104.812499 95.333749) (end 105.5625 96.08375) (width 0.25) (layer B.Cu) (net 3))
 (segment (start 104.812499 89.396251) (end 104.812499 95.333749) (width 0.25) (layer B.Cu) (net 3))
 (segment (start 105.5625 88.64625) (end 104.812499 89.396251) (width 0.25) (layer B.Cu) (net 3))
 (segment (start 105.5625 88.615) (end 105.5625 88.64625) (width 0.25) (layer B.Cu) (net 3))
 (segment (start 112.26 96.115) (end 113.18 95.195) (width 0.25) (layer B.Cu) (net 3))
 (segment (start 105.5625 96.115) (end 112.26 96.115) (width 0.25) (layer B.Cu) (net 3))
 (via (at 113.18 95.195) (size 0.8) (drill 0.4) (layers F.Cu B.Cu) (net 3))
 (segment (start 113.18 97.67) (end 113.18 95.195) (width 0.25) (layer F.Cu) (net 3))
 (segment (start 115.57 100.06) (end 113.18 97.67) (width 0.25) (layer F.Cu) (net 3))
 (segment (start 115.57 100.33) (end 115.57 100.06) (width 0.25) (layer F.Cu) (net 3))
 (via (at 115.57 100.33) (size 0.8) (drill 0.4) (layers F.Cu B.Cu) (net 3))
 (segment (start 115.855 100.615) (end 115.57 100.33) (width 0.25) (layer B.Cu) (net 3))
 (segment (start 119.38 97.59) (end 118.11 96.32) (width 0.25) (layer B.Cu) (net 3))
 (segment (start 119.38 100.615) (end 119.38 97.59) (width 0.25) (layer B.Cu) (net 3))
 (via (at 118.11 96.32) (size 0.8) (drill 0.4) (layers F.Cu B.Cu) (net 3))
 (segment (start 119.38 100.615) (end 115.855 100.615) (width 0.25) (layer B.Cu) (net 3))
 (segment (start 123.0375 100.615) (end 119.38 100.615) (width 0.25) (layer B.Cu) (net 3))
 (via (at 113.03 100.33) (size 0.8) (drill 0.4) (layers F.Cu B.Cu) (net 4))
 (segment (start 105.5625 97.615) (end 110.315 97.615) (width 0.25) (layer B.Cu) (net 4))
 (segment (start 110.315 97.615) (end 113.03 100.33) (width 0.25) (layer B.Cu) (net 4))
 (via (at 110.49 100.33) (size 0.8) (drill 0.4) (layers F.Cu B.Cu) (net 5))
 (segment (start 105.5625 99.115) (end 109.275 99.115) (width 0.25) (layer B.Cu) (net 5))
 (segment (start 109.275 99.115) (end 110.49 100.33) (width 0.25) (layer B.Cu) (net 5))
 (segment (start 117.800899 106.587584) (end 119.940889 104.447594) (width 0.25) (layer B.Cu) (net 8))
 (segment (start 119.940889 104.447594) (end 122.227594 104.447594) (width 0.25) (layer B.Cu) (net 8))
 (segment (start 122.227594 104.447594) (end 123.19 105.41) (width 0.25) (layer B.Cu) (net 8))
 (segment (start 125.268499 119.38) (end 125.420899 119.38) (width 0.25) (layer B.Cu) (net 8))
 (segment (start 123.19 117.301501) (end 125.268499 119.38) (width 0.25) (layer B.Cu) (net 8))
 (segment (start 123.19 105.41) (end 123.19 117.301501) (width 0.25) (layer B.Cu) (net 8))
 (segment (start 119.070899 121.92) (end 120.65 121.92) (width 0.25) (layer B.Cu) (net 13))
 (segment (start 120.65 121.92) (end 121.92 120.65) (width 0.25) (layer B.Cu) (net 13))
 (segment (start 121.92 120.65) (end 121.92 107.95) (width 0.25) (layer B.Cu) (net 13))
 (segment (start 121.703315 107.95) (end 120.340899 106.587584) (width 0.25) (layer B.Cu) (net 13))
 (segment (start 121.92 107.95) (end 121.703315 107.95) (width 0.25) (layer B.Cu) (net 13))
 (segment (start 112.720899 111.667584) (end 112.720899 106.587584) (width 0.25) (layer F.Cu) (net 14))
 (segment (start 110.180899 107.789665) (end 110.180899 111.667584) (width 0.25) (layer F.Cu) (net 15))
 (segment (start 110.180899 106.587584) (end 110.180899 107.789665) (width 0.25) (layer F.Cu) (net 15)))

